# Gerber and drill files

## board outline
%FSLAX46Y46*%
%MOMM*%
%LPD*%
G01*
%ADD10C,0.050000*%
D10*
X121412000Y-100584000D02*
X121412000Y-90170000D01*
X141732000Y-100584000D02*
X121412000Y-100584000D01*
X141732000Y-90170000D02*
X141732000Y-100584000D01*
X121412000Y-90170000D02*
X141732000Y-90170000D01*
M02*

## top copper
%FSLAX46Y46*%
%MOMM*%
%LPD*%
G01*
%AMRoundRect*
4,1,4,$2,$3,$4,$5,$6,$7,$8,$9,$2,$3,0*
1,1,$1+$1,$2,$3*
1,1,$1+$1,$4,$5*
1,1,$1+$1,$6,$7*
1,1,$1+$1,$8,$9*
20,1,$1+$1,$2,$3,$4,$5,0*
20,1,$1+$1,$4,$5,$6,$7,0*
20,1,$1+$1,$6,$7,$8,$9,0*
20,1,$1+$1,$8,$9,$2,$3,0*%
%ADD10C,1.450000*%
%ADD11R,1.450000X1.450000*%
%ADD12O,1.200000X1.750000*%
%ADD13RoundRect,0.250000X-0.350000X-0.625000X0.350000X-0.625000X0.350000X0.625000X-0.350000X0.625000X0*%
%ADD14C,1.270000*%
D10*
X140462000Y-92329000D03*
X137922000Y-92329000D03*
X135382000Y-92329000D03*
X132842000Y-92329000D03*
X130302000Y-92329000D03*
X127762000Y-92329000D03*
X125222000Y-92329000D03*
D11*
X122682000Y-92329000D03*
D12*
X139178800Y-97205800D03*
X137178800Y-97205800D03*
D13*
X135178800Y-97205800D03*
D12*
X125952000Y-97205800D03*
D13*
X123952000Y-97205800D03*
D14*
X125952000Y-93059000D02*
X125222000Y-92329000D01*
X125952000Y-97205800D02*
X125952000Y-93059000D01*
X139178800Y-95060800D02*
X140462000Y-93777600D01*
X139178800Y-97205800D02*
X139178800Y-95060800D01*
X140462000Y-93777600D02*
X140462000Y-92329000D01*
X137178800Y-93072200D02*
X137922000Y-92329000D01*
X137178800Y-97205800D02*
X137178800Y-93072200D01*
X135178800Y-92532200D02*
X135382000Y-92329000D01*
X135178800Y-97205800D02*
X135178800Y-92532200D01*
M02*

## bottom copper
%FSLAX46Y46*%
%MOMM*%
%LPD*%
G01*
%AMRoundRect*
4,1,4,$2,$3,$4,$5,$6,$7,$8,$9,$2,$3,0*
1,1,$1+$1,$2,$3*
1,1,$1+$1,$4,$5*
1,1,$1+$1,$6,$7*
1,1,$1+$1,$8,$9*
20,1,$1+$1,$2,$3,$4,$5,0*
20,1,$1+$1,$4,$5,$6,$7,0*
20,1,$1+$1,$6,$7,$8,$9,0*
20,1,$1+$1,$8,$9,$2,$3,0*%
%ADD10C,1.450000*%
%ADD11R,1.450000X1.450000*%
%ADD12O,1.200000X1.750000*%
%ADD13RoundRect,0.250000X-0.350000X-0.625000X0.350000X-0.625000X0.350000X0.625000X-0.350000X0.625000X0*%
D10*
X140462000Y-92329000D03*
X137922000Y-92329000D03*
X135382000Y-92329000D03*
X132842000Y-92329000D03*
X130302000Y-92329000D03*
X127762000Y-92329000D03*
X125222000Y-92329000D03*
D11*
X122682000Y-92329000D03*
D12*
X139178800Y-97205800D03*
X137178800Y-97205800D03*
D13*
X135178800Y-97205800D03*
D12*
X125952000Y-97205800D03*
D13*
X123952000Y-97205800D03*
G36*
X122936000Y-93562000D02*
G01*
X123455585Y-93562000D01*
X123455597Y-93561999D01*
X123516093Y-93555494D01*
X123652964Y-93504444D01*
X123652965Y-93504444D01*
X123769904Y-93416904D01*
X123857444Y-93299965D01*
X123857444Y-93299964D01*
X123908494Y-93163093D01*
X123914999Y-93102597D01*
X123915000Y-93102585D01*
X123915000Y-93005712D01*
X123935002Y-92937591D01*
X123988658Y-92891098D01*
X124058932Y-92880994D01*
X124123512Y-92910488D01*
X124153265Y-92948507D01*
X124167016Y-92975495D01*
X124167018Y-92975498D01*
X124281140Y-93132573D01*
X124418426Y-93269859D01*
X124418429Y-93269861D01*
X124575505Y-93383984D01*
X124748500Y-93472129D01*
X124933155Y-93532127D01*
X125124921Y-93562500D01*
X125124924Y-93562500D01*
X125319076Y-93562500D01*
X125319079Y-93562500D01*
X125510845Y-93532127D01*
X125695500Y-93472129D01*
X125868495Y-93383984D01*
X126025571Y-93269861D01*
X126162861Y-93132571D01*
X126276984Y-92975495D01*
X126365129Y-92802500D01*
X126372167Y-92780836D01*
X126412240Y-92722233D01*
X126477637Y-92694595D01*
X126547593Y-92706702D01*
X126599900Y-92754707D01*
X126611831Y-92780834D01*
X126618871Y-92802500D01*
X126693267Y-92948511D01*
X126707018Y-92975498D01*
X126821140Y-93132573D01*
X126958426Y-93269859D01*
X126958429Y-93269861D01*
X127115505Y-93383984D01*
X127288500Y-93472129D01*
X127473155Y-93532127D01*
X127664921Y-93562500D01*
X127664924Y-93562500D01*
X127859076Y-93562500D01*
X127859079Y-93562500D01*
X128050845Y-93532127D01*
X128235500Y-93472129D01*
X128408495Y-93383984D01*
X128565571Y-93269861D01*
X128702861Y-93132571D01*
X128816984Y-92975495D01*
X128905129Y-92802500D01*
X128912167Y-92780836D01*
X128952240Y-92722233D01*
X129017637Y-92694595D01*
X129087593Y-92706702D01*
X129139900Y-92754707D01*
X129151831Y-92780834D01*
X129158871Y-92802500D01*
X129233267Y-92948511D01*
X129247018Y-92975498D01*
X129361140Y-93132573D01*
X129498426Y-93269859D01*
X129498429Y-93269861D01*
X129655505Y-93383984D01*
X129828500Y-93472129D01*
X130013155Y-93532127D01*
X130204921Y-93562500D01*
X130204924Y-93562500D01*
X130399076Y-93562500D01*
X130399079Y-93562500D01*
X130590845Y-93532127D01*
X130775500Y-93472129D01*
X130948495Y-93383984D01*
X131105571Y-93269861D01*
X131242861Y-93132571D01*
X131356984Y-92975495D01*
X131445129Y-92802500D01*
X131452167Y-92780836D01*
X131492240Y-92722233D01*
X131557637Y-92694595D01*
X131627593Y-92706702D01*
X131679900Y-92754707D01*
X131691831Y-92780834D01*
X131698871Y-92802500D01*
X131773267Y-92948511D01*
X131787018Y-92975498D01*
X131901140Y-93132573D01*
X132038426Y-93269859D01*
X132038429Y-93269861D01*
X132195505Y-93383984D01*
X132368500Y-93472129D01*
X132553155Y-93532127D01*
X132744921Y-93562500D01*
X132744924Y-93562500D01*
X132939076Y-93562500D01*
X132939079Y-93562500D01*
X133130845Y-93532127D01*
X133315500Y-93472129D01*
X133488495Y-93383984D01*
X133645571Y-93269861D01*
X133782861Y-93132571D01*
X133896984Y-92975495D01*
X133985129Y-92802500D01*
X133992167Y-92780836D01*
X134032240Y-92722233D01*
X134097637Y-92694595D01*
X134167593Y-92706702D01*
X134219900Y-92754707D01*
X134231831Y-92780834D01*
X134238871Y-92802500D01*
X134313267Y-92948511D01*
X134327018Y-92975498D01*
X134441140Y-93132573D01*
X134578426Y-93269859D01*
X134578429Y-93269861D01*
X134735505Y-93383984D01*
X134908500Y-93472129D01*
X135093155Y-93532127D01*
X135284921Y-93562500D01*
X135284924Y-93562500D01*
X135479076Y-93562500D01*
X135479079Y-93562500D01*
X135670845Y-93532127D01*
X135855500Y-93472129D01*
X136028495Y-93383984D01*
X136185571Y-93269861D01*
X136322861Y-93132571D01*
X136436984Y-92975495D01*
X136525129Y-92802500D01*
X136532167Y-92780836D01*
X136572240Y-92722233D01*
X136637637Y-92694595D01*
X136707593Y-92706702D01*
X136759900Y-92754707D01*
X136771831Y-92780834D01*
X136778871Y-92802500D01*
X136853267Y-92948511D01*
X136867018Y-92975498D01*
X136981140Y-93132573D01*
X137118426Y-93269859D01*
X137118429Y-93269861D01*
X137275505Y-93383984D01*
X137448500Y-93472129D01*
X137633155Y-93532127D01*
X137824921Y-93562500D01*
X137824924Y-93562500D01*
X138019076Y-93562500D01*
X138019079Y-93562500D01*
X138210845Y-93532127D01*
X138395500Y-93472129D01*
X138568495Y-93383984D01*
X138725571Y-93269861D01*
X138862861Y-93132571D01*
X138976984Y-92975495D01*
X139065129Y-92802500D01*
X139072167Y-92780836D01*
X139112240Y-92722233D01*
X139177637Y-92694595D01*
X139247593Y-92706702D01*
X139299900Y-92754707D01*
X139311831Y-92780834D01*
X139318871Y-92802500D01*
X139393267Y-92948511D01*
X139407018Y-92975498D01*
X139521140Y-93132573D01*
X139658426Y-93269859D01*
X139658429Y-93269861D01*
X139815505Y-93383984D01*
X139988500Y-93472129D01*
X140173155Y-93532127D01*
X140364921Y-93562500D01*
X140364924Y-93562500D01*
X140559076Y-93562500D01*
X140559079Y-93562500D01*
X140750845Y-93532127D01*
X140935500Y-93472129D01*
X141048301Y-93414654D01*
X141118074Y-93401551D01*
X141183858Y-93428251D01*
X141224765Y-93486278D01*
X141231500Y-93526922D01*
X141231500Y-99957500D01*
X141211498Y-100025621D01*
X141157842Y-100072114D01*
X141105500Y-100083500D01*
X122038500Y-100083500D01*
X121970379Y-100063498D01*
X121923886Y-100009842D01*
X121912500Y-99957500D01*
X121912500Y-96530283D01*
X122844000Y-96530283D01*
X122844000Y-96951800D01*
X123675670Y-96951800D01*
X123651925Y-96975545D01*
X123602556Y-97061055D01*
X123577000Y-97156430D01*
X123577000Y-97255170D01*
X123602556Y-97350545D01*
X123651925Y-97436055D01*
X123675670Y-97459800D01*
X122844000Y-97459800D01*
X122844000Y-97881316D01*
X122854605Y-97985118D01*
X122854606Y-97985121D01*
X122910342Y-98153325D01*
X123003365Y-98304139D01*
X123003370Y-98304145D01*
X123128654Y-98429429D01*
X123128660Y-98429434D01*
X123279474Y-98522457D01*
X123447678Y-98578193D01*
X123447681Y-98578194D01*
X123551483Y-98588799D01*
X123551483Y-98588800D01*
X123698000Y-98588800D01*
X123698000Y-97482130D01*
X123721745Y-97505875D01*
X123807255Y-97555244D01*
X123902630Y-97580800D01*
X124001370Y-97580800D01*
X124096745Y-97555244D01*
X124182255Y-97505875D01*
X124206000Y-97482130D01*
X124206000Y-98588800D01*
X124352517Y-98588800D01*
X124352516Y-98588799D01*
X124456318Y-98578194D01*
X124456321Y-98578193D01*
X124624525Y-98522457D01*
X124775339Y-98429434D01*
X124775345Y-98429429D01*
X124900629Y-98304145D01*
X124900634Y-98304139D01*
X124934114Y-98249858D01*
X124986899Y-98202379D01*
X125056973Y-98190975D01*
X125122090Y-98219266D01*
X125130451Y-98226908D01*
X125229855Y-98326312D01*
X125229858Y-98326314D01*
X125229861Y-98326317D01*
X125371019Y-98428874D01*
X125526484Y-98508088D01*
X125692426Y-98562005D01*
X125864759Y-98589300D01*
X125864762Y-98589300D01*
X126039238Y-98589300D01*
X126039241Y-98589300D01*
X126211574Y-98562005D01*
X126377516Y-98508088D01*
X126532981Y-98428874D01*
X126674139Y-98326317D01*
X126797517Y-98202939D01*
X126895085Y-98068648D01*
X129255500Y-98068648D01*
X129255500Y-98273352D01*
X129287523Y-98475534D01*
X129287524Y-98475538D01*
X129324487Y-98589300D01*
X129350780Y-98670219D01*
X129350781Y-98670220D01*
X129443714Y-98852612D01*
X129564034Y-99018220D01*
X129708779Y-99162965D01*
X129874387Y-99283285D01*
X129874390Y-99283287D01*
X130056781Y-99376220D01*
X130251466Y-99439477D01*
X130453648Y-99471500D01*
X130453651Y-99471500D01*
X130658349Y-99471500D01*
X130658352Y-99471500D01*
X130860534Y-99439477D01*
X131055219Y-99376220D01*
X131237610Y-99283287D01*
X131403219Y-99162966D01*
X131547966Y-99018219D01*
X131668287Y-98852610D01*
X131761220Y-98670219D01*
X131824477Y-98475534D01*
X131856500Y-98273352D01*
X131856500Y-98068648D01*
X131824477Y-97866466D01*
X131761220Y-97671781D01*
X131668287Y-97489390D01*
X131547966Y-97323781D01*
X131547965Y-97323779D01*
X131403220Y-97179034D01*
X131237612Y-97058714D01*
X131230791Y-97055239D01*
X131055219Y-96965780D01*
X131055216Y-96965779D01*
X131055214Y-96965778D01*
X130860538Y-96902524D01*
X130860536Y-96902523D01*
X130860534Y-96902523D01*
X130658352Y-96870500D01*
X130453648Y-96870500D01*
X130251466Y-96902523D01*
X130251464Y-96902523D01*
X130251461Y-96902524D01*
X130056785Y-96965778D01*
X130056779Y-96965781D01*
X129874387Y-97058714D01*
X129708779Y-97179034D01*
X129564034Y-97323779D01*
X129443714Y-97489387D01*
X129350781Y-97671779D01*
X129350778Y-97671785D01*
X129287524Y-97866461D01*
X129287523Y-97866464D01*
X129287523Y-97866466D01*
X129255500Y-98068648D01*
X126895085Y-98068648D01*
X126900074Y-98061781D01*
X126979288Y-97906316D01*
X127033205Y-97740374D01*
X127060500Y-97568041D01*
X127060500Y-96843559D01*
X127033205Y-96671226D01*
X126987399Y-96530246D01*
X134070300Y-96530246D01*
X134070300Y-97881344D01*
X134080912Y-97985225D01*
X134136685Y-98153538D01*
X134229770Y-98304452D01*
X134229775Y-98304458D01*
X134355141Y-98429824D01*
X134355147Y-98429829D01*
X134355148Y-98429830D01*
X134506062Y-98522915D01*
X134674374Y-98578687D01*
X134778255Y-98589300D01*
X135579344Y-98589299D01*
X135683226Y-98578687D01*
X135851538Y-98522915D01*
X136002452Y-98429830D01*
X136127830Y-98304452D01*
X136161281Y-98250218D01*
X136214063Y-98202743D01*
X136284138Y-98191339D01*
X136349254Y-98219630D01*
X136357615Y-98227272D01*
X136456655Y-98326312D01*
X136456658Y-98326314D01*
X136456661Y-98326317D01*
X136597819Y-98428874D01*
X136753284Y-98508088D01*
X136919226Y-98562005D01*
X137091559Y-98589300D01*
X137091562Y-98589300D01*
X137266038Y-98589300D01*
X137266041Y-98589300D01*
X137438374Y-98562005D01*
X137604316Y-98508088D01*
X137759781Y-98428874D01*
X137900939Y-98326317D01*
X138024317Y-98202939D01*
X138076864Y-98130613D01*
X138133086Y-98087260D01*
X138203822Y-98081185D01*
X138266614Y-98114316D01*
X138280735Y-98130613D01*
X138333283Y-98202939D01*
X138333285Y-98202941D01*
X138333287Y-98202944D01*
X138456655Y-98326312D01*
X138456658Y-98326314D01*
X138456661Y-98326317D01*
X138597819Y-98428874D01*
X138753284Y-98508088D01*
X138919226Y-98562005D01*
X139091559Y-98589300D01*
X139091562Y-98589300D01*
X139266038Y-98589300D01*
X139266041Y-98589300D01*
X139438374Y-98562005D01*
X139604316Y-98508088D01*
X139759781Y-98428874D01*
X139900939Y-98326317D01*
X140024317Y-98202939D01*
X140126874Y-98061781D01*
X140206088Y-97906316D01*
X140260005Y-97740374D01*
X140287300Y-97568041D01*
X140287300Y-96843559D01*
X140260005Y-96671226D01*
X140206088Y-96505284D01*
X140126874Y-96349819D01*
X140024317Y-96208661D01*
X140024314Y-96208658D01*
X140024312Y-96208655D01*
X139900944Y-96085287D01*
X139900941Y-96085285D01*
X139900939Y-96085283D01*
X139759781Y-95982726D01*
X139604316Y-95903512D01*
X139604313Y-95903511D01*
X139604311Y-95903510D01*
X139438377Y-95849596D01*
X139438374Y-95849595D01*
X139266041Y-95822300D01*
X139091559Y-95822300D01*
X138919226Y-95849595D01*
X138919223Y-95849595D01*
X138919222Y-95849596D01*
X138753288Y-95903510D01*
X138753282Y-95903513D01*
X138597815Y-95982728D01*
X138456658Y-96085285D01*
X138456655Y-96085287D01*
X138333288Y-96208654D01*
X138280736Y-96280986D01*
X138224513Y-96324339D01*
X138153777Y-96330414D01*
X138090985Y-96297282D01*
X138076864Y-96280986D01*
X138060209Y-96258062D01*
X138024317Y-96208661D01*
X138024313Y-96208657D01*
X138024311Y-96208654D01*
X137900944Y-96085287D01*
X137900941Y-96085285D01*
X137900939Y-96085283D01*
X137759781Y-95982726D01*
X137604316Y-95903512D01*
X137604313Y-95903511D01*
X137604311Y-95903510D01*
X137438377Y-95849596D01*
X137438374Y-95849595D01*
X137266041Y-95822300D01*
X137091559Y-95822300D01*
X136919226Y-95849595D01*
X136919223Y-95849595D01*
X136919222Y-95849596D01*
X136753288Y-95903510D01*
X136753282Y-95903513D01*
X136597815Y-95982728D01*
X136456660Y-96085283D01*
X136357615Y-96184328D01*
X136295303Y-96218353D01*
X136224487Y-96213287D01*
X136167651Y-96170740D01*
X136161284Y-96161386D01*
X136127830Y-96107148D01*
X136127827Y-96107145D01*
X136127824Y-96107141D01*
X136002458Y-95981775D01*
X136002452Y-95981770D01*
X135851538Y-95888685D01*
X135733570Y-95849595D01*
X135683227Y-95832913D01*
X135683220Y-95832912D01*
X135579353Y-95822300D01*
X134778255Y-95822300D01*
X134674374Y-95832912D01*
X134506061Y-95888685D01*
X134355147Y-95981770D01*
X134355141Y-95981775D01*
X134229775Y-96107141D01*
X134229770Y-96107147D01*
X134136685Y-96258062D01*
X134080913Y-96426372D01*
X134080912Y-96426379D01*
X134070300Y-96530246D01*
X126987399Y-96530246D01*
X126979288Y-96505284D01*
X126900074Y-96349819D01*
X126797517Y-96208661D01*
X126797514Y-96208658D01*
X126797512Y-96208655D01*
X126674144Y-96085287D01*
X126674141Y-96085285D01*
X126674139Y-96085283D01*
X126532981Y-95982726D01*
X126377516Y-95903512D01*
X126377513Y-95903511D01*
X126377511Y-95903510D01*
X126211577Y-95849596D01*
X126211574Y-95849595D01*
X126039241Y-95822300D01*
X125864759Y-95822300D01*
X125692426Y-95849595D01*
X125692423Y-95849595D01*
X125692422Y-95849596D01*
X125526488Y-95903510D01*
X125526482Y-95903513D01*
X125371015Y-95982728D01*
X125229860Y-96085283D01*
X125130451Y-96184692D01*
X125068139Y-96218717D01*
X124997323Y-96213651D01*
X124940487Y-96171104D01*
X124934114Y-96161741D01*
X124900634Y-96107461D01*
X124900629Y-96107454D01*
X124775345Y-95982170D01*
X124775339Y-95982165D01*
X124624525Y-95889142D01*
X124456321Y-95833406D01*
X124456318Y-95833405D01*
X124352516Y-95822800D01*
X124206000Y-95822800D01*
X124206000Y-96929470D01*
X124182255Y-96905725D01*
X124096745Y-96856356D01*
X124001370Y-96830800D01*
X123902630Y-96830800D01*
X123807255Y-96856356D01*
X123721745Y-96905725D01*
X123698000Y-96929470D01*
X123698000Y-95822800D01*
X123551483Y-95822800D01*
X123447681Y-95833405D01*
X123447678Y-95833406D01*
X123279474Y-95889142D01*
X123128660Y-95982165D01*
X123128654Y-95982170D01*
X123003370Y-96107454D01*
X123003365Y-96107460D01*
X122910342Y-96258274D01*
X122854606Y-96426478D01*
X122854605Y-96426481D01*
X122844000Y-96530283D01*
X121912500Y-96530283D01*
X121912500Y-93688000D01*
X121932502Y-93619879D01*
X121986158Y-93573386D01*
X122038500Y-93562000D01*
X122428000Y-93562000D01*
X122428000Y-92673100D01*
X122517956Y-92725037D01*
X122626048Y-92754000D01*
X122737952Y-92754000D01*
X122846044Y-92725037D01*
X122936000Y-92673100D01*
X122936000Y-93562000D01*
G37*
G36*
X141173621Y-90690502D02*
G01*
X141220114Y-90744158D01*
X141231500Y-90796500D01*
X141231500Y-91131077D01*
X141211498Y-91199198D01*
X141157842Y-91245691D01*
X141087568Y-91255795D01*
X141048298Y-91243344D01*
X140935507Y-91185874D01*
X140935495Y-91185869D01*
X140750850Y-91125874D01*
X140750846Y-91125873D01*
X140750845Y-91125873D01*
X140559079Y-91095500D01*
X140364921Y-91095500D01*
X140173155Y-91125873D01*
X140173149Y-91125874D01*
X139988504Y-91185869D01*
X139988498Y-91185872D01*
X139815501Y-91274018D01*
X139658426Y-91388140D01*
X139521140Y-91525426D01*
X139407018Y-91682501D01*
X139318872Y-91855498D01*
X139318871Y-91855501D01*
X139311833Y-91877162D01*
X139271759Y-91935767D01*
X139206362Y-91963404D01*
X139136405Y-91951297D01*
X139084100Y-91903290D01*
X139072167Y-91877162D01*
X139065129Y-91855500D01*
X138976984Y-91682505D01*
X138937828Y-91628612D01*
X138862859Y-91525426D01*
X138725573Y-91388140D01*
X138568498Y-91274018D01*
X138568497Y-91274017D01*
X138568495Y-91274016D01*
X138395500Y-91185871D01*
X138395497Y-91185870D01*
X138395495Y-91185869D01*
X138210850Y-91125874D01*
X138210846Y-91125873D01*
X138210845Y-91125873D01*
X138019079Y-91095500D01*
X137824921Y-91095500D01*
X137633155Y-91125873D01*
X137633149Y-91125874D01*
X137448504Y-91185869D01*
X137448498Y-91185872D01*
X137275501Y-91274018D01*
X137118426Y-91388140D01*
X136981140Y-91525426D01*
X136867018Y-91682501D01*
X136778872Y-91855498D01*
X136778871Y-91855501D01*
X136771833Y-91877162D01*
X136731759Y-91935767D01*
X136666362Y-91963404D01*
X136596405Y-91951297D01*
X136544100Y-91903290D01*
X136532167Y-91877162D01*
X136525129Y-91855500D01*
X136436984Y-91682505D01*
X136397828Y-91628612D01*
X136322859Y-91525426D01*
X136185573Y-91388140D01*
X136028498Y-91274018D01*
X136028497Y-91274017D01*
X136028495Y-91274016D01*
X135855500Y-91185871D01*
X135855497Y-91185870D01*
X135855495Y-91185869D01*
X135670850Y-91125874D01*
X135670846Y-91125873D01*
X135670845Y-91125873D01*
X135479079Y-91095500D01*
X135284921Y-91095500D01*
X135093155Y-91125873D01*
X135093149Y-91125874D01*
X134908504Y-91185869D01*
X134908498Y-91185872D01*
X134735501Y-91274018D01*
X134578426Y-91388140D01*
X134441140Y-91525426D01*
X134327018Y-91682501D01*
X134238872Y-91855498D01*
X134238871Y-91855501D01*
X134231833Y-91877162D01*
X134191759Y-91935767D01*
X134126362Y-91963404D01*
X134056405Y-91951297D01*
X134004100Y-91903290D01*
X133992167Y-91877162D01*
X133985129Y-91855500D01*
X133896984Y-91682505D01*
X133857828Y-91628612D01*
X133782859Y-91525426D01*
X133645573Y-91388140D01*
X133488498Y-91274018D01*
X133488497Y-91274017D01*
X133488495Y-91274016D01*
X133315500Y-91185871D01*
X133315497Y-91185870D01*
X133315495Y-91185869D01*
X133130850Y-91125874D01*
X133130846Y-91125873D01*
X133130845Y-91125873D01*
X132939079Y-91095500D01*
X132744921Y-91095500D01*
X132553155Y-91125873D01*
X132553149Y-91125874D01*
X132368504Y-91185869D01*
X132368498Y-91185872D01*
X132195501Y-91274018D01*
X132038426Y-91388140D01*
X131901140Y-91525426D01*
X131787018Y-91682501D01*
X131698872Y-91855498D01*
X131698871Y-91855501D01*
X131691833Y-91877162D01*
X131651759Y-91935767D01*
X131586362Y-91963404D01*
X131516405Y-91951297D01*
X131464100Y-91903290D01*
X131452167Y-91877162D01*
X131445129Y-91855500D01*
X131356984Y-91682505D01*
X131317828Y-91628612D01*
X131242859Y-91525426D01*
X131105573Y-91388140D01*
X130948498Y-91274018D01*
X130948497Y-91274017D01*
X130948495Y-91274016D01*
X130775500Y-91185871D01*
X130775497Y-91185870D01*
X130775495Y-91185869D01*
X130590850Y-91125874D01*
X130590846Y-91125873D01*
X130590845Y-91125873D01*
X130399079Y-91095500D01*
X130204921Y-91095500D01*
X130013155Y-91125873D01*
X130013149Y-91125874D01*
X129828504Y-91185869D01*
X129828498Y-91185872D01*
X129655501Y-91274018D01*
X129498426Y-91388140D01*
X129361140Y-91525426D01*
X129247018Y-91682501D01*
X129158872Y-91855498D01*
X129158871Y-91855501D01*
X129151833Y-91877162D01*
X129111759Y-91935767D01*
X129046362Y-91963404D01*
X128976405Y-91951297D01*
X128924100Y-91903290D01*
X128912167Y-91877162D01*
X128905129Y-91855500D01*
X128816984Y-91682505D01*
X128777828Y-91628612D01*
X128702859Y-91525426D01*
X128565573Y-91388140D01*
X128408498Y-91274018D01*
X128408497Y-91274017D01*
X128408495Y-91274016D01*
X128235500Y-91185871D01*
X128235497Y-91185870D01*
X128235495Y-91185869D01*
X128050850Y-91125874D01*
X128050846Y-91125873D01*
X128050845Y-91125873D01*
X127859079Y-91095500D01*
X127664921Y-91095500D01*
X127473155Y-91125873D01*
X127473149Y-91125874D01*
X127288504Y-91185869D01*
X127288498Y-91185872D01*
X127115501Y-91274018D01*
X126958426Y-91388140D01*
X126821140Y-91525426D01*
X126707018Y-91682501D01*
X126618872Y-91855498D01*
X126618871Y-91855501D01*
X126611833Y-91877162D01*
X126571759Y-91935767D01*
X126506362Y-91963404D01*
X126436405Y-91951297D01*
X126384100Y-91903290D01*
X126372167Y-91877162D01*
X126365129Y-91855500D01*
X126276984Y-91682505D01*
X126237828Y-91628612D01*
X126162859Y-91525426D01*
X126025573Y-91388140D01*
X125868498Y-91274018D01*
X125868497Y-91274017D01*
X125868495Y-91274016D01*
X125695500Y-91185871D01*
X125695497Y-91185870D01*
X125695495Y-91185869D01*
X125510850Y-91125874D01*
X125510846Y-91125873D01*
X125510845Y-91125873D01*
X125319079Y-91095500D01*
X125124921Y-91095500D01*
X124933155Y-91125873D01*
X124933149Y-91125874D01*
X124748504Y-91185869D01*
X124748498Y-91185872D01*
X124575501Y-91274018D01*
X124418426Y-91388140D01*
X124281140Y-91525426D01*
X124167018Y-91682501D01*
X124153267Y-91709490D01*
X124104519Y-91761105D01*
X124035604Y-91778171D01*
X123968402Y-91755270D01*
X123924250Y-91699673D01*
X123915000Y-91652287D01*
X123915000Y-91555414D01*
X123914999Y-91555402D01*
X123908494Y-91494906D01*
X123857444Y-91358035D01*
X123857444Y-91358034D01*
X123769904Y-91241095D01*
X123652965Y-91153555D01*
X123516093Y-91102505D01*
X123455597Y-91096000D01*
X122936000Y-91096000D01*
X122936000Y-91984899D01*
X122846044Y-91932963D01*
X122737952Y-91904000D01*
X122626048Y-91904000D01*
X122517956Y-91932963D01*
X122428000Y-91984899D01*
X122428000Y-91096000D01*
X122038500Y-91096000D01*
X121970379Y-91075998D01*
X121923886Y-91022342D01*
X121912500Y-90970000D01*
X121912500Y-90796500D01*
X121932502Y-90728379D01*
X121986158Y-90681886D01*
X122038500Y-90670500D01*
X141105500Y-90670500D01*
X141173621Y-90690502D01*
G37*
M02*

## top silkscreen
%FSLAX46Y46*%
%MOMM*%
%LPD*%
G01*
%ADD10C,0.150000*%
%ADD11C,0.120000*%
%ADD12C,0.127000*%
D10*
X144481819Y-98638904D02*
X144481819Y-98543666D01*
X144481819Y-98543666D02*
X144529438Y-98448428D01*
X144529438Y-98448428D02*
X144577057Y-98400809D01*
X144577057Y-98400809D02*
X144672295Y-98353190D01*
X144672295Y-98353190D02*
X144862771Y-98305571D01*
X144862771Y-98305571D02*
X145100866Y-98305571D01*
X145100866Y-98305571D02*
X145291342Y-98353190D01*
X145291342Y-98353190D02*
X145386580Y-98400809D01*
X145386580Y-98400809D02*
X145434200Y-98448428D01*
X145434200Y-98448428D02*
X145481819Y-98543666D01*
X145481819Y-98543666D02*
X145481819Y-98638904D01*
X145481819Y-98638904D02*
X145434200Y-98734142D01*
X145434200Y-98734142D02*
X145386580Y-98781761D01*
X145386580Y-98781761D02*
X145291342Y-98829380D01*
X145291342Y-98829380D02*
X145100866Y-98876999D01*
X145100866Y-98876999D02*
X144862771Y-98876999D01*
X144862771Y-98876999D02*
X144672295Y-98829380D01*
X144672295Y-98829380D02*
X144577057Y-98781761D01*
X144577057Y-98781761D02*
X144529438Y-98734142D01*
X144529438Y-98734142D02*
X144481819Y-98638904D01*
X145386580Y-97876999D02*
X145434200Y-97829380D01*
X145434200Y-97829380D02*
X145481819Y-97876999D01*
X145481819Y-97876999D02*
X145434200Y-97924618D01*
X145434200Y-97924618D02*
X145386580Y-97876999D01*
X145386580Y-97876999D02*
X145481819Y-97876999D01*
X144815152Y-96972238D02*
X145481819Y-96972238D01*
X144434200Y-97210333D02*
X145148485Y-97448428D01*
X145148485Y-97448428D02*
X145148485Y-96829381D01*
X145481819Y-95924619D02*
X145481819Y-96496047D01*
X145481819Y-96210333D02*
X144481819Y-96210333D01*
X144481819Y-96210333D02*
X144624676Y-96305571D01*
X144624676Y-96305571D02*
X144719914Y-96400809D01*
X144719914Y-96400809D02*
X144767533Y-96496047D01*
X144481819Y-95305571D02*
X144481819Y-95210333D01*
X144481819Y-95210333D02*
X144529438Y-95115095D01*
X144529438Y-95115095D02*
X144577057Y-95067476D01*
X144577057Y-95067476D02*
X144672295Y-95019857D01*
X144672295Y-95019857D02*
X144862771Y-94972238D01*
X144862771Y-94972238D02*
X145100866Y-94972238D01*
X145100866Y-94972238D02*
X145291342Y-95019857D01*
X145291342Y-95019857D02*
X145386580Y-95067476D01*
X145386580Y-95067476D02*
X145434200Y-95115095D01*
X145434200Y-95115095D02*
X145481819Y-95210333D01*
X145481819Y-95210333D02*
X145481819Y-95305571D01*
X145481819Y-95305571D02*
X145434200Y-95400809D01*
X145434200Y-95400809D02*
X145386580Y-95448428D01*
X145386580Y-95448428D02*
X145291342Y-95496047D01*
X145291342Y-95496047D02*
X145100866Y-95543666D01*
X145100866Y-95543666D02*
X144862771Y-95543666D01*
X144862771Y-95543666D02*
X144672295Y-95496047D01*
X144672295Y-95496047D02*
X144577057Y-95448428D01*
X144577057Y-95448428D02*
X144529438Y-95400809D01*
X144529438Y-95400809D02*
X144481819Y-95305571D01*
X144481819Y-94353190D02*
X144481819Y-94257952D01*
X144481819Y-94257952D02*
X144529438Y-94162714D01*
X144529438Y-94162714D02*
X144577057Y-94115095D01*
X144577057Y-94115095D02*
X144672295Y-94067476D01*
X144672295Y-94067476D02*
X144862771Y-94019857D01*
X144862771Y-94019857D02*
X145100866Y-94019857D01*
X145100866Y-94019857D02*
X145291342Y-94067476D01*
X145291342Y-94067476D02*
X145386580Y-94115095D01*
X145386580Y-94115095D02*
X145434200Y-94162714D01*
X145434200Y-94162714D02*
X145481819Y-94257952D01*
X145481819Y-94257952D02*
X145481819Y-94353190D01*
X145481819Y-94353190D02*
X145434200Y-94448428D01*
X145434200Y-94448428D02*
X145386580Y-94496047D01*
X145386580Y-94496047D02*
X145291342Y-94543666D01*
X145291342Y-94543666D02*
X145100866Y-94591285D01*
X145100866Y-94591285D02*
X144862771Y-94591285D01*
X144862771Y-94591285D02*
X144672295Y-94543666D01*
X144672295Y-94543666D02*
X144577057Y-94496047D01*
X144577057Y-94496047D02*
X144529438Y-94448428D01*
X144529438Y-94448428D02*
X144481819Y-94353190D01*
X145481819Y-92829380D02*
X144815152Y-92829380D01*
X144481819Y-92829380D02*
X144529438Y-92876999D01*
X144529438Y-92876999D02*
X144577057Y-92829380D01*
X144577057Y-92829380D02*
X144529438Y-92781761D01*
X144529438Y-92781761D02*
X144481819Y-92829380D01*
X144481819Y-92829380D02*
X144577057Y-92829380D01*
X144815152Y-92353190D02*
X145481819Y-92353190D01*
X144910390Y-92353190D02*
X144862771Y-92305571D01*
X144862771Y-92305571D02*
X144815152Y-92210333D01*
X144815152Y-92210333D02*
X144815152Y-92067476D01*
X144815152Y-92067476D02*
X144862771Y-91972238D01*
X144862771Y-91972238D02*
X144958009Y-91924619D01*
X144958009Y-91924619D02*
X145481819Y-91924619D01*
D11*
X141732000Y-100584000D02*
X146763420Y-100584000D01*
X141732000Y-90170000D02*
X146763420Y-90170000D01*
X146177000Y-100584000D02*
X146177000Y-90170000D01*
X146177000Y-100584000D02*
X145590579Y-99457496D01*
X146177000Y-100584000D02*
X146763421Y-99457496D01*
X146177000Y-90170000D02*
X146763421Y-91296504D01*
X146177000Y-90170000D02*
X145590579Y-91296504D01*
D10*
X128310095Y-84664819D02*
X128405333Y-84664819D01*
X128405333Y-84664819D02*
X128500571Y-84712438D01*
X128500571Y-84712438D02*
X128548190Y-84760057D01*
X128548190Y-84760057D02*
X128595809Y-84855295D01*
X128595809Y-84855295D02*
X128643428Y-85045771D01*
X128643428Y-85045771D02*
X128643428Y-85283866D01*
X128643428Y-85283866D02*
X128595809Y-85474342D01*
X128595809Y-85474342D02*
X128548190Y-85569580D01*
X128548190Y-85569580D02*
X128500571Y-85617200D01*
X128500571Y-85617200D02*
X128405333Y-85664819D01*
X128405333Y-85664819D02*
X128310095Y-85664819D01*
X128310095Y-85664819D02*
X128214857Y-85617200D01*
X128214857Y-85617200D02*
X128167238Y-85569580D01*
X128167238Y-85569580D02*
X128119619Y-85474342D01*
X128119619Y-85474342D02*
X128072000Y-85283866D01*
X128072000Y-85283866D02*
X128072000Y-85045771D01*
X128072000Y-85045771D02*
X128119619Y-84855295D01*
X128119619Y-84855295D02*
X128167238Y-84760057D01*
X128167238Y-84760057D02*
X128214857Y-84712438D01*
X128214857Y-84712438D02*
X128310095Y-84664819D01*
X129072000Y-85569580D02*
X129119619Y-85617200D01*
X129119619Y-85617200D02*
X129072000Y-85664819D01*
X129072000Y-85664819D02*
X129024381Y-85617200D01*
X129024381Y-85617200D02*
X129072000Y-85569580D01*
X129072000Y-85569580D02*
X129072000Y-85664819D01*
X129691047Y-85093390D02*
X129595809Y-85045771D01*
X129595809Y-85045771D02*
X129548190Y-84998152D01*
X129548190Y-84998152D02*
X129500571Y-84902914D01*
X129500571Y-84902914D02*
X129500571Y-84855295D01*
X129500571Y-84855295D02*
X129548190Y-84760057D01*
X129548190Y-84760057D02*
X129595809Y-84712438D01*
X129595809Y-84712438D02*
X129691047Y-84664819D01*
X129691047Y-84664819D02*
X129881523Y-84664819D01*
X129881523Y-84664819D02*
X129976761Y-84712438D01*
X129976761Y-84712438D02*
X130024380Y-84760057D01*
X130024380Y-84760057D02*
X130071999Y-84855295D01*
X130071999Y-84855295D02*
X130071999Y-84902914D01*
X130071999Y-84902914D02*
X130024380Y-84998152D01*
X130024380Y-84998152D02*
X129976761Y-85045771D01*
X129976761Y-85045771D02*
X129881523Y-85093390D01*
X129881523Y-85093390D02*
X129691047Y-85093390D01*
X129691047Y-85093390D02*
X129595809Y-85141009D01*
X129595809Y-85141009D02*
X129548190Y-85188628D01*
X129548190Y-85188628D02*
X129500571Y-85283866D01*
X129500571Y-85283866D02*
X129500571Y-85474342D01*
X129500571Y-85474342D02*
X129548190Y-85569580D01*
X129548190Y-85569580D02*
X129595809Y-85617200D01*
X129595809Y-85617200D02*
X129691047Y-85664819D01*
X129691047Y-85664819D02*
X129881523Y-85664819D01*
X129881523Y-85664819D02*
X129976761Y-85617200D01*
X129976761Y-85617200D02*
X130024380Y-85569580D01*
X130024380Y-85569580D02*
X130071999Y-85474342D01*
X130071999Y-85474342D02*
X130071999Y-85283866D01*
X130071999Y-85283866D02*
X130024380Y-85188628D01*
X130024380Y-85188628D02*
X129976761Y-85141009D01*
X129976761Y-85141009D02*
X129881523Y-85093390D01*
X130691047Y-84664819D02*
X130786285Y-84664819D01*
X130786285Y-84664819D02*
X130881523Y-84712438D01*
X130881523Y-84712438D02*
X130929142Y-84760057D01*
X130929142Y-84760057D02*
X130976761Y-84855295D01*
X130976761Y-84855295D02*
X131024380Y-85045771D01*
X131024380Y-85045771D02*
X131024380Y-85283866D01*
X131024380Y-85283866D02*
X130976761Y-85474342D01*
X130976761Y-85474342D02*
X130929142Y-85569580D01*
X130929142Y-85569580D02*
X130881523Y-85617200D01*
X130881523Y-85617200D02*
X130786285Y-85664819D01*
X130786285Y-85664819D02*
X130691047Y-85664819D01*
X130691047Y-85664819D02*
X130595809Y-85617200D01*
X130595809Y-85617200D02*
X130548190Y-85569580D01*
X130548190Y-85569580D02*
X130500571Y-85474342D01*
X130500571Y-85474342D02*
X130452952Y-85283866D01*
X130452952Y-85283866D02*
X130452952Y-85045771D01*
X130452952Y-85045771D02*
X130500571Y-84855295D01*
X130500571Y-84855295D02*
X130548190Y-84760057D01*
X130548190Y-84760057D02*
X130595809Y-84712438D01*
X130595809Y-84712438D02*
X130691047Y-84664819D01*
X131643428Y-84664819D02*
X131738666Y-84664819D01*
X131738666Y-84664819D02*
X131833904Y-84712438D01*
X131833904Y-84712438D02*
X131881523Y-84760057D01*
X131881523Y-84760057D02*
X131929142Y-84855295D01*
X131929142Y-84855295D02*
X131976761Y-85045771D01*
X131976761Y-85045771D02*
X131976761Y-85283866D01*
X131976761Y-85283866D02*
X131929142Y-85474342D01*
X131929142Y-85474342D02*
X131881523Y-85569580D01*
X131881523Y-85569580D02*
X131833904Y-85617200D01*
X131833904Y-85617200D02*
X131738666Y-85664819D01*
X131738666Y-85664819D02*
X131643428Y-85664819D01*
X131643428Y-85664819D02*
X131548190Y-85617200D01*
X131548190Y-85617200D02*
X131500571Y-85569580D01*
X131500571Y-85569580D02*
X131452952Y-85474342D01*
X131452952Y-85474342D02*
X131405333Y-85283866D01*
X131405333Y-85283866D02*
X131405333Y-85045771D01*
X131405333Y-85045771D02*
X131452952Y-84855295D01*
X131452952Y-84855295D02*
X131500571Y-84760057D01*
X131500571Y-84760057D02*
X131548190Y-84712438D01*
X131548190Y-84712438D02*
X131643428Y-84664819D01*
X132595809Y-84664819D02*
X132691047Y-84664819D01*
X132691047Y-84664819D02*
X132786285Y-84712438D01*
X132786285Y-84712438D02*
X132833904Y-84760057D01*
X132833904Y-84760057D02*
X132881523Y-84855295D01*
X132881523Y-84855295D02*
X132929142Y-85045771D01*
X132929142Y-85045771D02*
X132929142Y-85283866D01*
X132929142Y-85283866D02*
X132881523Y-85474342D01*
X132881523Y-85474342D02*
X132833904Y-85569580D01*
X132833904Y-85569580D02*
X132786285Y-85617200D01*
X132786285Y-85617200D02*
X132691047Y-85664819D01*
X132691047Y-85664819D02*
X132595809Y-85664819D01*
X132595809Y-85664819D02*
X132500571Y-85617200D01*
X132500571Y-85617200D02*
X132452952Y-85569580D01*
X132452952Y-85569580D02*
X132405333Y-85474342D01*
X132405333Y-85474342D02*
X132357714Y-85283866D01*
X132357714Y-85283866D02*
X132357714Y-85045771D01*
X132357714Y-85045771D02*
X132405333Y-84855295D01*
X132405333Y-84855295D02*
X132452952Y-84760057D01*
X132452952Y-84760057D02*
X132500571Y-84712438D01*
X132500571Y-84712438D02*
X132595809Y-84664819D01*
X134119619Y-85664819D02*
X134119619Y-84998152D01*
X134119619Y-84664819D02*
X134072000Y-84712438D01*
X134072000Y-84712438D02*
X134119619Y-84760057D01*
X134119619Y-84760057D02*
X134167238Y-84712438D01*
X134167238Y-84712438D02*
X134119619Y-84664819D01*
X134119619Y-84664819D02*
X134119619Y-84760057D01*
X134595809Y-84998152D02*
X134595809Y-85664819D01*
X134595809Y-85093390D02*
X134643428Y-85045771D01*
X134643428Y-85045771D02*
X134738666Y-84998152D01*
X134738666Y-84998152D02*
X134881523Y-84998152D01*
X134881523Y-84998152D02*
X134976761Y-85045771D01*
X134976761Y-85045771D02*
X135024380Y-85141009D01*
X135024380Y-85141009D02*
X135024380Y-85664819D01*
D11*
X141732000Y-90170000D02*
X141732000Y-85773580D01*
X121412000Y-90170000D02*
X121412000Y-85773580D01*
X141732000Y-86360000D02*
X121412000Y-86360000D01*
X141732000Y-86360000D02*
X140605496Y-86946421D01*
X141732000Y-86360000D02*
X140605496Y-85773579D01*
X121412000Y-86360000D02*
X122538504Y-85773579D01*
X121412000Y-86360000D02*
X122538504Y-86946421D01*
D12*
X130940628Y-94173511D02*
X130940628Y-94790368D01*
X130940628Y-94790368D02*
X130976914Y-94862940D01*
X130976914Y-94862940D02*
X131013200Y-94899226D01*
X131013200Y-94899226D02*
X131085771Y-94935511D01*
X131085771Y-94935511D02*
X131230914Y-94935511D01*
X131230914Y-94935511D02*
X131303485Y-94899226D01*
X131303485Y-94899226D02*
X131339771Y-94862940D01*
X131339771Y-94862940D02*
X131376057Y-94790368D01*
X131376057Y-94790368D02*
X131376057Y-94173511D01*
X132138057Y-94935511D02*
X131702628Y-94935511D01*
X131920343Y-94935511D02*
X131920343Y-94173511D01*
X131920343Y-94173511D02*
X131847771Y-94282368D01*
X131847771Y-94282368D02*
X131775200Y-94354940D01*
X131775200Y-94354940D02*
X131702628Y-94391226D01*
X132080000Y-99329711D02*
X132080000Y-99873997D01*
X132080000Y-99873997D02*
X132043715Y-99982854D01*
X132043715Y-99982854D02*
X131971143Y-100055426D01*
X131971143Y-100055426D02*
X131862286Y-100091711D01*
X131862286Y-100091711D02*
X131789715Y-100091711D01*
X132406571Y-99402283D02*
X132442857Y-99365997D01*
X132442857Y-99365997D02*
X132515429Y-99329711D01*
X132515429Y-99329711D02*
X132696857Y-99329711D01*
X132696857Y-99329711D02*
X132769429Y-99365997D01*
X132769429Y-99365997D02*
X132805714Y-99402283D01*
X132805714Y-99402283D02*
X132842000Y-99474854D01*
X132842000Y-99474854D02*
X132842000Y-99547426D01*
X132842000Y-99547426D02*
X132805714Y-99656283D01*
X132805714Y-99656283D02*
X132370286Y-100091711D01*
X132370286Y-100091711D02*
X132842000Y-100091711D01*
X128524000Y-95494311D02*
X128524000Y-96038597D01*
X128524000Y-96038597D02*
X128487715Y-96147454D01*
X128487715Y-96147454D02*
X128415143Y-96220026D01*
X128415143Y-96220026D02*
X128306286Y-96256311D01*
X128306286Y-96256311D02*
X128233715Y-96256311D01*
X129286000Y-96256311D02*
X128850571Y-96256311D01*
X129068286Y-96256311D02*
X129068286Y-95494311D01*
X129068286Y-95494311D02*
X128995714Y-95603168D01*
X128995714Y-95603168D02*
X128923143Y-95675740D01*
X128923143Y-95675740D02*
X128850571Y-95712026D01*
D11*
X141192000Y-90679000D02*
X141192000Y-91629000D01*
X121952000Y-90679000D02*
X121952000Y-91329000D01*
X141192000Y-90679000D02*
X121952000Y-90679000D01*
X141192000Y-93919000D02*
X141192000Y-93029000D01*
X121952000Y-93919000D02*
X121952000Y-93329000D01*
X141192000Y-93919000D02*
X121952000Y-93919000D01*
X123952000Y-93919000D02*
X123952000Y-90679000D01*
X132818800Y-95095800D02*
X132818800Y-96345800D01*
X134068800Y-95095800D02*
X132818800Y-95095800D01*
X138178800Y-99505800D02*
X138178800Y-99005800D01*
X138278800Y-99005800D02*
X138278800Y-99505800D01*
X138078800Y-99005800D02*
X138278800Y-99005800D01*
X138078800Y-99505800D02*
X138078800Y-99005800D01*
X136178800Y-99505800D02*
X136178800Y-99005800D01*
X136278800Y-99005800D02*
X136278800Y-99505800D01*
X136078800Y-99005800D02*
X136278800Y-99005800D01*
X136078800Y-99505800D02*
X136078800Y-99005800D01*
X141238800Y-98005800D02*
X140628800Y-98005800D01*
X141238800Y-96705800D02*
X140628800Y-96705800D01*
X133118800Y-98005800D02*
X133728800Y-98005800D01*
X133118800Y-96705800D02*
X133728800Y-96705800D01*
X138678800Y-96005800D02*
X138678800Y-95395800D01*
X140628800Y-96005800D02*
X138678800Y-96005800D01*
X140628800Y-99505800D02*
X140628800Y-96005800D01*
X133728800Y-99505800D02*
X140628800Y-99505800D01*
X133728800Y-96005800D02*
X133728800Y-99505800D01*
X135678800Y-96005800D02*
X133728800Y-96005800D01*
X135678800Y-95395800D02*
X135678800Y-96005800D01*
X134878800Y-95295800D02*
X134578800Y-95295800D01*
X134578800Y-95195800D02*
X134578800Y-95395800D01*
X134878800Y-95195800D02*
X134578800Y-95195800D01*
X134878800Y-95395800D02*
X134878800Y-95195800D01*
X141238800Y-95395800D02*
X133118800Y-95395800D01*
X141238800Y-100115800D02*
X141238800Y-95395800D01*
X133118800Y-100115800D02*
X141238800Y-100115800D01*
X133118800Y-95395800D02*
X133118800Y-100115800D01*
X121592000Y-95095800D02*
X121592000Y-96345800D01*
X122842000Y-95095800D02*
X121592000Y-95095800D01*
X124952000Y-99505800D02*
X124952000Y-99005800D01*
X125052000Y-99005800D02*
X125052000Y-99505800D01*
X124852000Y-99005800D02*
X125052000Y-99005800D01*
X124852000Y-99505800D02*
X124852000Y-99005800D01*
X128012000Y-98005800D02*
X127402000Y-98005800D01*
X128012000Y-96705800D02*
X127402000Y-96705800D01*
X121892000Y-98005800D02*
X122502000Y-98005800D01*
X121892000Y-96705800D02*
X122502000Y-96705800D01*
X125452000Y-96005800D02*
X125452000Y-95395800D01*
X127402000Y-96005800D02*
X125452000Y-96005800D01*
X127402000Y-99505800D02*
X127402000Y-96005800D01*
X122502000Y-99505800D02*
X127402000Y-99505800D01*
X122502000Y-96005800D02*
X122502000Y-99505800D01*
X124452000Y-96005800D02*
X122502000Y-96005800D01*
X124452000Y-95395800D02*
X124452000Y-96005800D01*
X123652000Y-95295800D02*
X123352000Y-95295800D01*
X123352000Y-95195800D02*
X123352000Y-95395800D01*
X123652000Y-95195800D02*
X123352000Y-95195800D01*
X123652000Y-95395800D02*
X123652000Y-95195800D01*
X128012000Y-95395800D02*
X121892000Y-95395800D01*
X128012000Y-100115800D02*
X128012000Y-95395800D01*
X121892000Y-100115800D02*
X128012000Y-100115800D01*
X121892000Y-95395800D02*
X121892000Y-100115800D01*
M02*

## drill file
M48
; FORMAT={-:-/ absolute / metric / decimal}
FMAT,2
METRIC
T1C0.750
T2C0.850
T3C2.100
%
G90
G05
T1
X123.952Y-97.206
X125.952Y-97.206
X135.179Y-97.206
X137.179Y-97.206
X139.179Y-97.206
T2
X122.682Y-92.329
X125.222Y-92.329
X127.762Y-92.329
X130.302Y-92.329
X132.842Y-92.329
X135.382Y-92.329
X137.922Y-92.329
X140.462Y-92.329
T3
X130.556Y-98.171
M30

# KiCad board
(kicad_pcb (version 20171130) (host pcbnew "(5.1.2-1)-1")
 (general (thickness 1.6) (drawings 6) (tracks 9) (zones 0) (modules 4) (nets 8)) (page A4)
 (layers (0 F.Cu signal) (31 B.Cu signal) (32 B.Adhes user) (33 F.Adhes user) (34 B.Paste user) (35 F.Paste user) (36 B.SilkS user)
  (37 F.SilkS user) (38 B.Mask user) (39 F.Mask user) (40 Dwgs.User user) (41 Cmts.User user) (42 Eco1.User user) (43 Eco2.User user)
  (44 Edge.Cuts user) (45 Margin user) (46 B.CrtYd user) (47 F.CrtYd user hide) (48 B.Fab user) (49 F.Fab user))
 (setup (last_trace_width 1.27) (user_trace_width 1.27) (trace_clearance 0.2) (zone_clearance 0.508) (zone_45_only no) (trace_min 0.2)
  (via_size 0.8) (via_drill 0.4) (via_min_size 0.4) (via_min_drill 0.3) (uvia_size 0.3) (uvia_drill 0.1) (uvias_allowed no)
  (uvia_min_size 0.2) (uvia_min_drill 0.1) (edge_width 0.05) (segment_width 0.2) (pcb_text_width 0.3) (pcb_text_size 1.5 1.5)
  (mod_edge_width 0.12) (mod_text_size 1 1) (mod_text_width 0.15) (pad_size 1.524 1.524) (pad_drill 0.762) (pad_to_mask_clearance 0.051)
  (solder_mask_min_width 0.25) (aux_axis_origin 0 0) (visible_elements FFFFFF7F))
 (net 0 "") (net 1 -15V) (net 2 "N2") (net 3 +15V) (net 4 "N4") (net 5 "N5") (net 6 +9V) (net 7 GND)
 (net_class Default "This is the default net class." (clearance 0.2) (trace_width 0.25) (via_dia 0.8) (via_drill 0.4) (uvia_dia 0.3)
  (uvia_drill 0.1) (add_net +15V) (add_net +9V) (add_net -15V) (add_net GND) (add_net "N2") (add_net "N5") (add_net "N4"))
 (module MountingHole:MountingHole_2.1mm (layer F.Cu) (at 130.556 98.171)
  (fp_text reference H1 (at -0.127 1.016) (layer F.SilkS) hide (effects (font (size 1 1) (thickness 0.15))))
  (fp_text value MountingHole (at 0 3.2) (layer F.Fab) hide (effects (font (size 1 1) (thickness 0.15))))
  (pad "" np_thru_hole circle (at 0 0) (size 2.1 2.1) (drill 2.1) (layers *.Cu *.Mask)))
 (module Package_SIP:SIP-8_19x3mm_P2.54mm (layer F.Cu) (at 122.682 92.329)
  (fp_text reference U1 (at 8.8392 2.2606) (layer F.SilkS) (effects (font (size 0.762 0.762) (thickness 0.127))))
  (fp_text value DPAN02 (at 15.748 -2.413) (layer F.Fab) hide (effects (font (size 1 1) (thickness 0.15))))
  (fp_line (start 18.51 -1.65) (end 18.51 -0.7) (layer F.SilkS) (width 0.12))
  (fp_line (start -0.73 -1.65) (end -0.73 -1) (layer F.SilkS) (width 0.12))
  (fp_line (start 18.51 -1.65) (end -0.73 -1.65) (layer F.SilkS) (width 0.12))
  (fp_line (start 18.51 1.59) (end 18.51 0.7) (layer F.SilkS) (width 0.12))
  (fp_line (start -0.73 1.59) (end -0.73 1) (layer F.SilkS) (width 0.12))
  (fp_line (start 18.51 1.59) (end -0.73 1.59) (layer F.SilkS) (width 0.12))
  (fp_line (start 1.27 1.59) (end 1.27 -1.65) (layer F.SilkS) (width 0.12))
  (pad 8 thru_hole circle (at 17.78 0 90) (size 1.45 1.45) (drill 0.85) (layers *.Cu *.Mask) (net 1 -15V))
  (pad 7 thru_hole circle (at 15.24 0 90) (size 1.45 1.45) (drill 0.85) (layers *.Cu *.Mask) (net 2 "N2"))
  (pad 6 thru_hole circle (at 12.7 0 90) (size 1.45 1.45) (drill 0.85) (layers *.Cu *.Mask) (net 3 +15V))
  (pad 5 thru_hole circle (at 10.16 0 90) (size 1.45 1.45) (drill 0.85) (layers *.Cu *.Mask) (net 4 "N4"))
  (pad 4 thru_hole circle (at 7.62 0 90) (size 1.45 1.45) (drill 0.85) (layers *.Cu *.Mask))
  (pad 3 thru_hole circle (at 5.08 0 90) (size 1.45 1.45) (drill 0.85) (layers *.Cu *.Mask) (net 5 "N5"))
  (pad 2 thru_hole circle (at 2.54 0 90) (size 1.45 1.45) (drill 0.85) (layers *.Cu *.Mask) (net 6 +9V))
  (pad 1 thru_hole rect (at 0 0 90) (size 1.45 1.45) (drill 0.85) (layers *.Cu *.Mask) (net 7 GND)))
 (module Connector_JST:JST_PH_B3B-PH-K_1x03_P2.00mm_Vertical (layer F.Cu) (at 135.1788 97.2058)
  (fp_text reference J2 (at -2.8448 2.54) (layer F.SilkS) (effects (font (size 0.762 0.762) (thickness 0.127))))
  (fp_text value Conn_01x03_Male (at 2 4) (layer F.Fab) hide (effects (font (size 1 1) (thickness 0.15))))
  (fp_line (start -2.36 -2.11) (end -2.36 -0.86) (layer F.SilkS) (width 0.12))
  (fp_line (start -1.11 -2.11) (end -2.36 -2.11) (layer F.SilkS) (width 0.12))
  (fp_line (start 3 2.3) (end 3 1.8) (layer F.SilkS) (width 0.12))
  (fp_line (start 3.1 1.8) (end 3.1 2.3) (layer F.SilkS) (width 0.12))
  (fp_line (start 2.9 1.8) (end 3.1 1.8) (layer F.SilkS) (width 0.12))
  (fp_line (start 2.9 2.3) (end 2.9 1.8) (layer F.SilkS) (width 0.12))
  (fp_line (start 1 2.3) (end 1 1.8) (layer F.SilkS) (width 0.12))
  (fp_line (start 1.1 1.8) (end 1.1 2.3) (layer F.SilkS) (width 0.12))
  (fp_line (start 0.9 1.8) (end 1.1 1.8) (layer F.SilkS) (width 0.12))
  (fp_line (start 0.9 2.3) (end 0.9 1.8) (layer F.SilkS) (width 0.12))
  (fp_line (start 6.06 0.8) (end 5.45 0.8) (layer F.SilkS) (width 0.12))
  (fp_line (start 6.06 -0.5) (end 5.45 -0.5) (layer F.SilkS) (width 0.12))
  (fp_line (start -2.06 0.8) (end -1.45 0.8) (layer F.SilkS) (width 0.12))
  (fp_line (start -2.06 -0.5) (end -1.45 -0.5) (layer F.SilkS) (width 0.12))
  (fp_line (start 3.5 -1.2) (end 3.5 -1.81) (layer F.SilkS) (width 0.12))
  (fp_line (start 5.45 -1.2) (end 3.5 -1.2) (layer F.SilkS) (width 0.12))
  (fp_line (start 5.45 2.3) (end 5.45 -1.2) (layer F.SilkS) (width 0.12))
  (fp_line (start -1.45 2.3) (end 5.45 2.3) (layer F.SilkS) (width 0.12))
  (fp_line (start -1.45 -1.2) (end -1.45 2.3) (layer F.SilkS) (width 0.12))
  (fp_line (start 0.5 -1.2) (end -1.45 -1.2) (layer F.SilkS) (width 0.12))
  (fp_line (start 0.5 -1.81) (end 0.5 -1.2) (layer F.SilkS) (width 0.12))
  (fp_line (start -0.3 -1.91) (end -0.6 -1.91) (layer F.SilkS) (width 0.12))
  (fp_line (start -0.6 -2.01) (end -0.6 -1.81) (layer F.SilkS) (width 0.12))
  (fp_line (start -0.3 -2.01) (end -0.6 -2.01) (layer F.SilkS) (width 0.12))
  (fp_line (start -0.3 -1.81) (end -0.3 -2.01) (layer F.SilkS) (width 0.12))
  (fp_line (start 6.06 -1.81) (end -2.06 -1.81) (layer F.SilkS) (width 0.12))
  (fp_line (start 6.06 2.91) (end 6.06 -1.81) (layer F.SilkS) (width 0.12))
  (fp_line (start -2.06 2.91) (end 6.06 2.91) (layer F.SilkS) (width 0.12))
  (fp_line (start -2.06 -1.81) (end -2.06 2.91) (layer F.SilkS) (width 0.12))
  (pad 3 thru_hole oval (at 4 0) (size 1.2 1.75) (drill 0.75) (layers *.Cu *.Mask) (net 1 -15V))
  (pad 2 thru_hole oval (at 2 0) (size 1.2 1.75) (drill 0.75) (layers *.Cu *.Mask) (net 2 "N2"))
  (pad 1 thru_hole roundrect (at 0 0) (size 1.2 1.75) (drill 0.75) (layers *.Cu *.Mask) (roundrect_rratio 0.208333) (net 3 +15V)))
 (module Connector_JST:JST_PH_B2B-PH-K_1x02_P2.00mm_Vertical (layer F.Cu) (at 123.952 97.2058)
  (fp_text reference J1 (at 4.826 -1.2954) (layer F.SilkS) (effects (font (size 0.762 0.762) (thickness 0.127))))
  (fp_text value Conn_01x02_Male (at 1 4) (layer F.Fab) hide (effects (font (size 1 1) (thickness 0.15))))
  (fp_line (start -2.36 -2.11) (end -2.36 -0.86) (layer F.SilkS) (width 0.12))
  (fp_line (start -1.11 -2.11) (end -2.36 -2.11) (layer F.SilkS) (width 0.12))
  (fp_line (start 1 2.3) (end 1 1.8) (layer F.SilkS) (width 0.12))
  (fp_line (start 1.1 1.8) (end 1.1 2.3) (layer F.SilkS) (width 0.12))
  (fp_line (start 0.9 1.8) (end 1.1 1.8) (layer F.SilkS) (width 0.12))
  (fp_line (start 0.9 2.3) (end 0.9 1.8) (layer F.SilkS) (width 0.12))
  (fp_line (start 4.06 0.8) (end 3.45 0.8) (layer F.SilkS) (width 0.12))
  (fp_line (start 4.06 -0.5) (end 3.45 -0.5) (layer F.SilkS) (width 0.12))
  (fp_line (start -2.06 0.8) (end -1.45 0.8) (layer F.SilkS) (width 0.12))
  (fp_line (start -2.06 -0.5) (end -1.45 -0.5) (layer F.SilkS) (width 0.12))
  (fp_line (start 1.5 -1.2) (end 1.5 -1.81) (layer F.SilkS) (width 0.12))
  (fp_line (start 3.45 -1.2) (end 1.5 -1.2) (layer F.SilkS) (width 0.12))
  (fp_line (start 3.45 2.3) (end 3.45 -1.2) (layer F.SilkS) (width 0.12))
  (fp_line (start -1.45 2.3) (end 3.45 2.3) (layer F.SilkS) (width 0.12))
  (fp_line (start -1.45 -1.2) (end -1.45 2.3) (layer F.SilkS) (width 0.12))
  (fp_line (start 0.5 -1.2) (end -1.45 -1.2) (layer F.SilkS) (width 0.12))
  (fp_line (start 0.5 -1.81) (end 0.5 -1.2) (layer F.SilkS) (width 0.12))
  (fp_line (start -0.3 -1.91) (end -0.6 -1.91) (layer F.SilkS) (width 0.12))
  (fp_line (start -0.6 -2.01) (end -0.6 -1.81) (layer F.SilkS) (width 0.12))
  (fp_line (start -0.3 -2.01) (end -0.6 -2.01) (layer F.SilkS) (width 0.12))
  (fp_line (start -0.3 -1.81) (end -0.3 -2.01) (layer F.SilkS) (width 0.12))
  (fp_line (start 4.06 -1.81) (end -2.06 -1.81) (layer F.SilkS) (width 0.12))
  (fp_line (start 4.06 2.91) (end 4.06 -1.81) (layer F.SilkS) (width 0.12))
  (fp_line (start -2.06 2.91) (end 4.06 2.91) (layer F.SilkS) (width 0.12))
  (fp_line (start -2.06 -1.81) (end -2.06 2.91) (layer F.SilkS) (width 0.12))
  (pad 2 thru_hole oval (at 2 0) (size 1.2 1.75) (drill 0.75) (layers *.Cu *.Mask) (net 6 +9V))
  (pad 1 thru_hole roundrect (at 0 0) (size 1.2 1.75) (drill 0.75) (layers *.Cu *.Mask) (roundrect_rratio 0.208333) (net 7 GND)))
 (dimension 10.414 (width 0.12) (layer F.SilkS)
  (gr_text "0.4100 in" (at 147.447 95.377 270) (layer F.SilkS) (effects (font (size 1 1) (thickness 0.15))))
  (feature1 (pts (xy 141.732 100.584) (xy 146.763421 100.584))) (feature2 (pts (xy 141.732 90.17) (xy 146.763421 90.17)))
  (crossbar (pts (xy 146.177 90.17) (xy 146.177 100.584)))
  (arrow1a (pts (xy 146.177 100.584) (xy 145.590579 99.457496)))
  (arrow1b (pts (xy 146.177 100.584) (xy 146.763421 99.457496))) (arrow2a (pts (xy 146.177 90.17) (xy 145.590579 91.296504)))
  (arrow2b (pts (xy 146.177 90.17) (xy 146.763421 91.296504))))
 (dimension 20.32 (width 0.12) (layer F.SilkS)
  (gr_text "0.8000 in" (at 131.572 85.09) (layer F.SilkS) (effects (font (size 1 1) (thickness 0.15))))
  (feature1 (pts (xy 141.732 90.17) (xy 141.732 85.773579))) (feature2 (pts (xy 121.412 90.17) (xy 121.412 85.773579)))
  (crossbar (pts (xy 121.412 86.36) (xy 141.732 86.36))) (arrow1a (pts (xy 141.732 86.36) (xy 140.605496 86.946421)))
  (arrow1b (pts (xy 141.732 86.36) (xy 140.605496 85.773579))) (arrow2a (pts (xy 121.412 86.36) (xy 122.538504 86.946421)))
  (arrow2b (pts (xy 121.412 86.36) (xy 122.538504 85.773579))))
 (gr_line (start 121.412 100.584) (end 121.412 90.17) (layer Edge.Cuts) (width 0.05))
 (gr_line (start 141.732 100.584) (end 121.412 100.584) (layer Edge.Cuts) (width 0.05))
 (gr_line (start 141.732 90.17) (end 141.732 100.584) (layer Edge.Cuts) (width 0.05))
 (gr_line (start 121.412 90.17) (end 141.732 90.17) (layer Edge.Cuts) (width 0.05))
 (segment (start 125.952 93.059) (end 125.222 92.329) (width 1.27) (layer F.Cu) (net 6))
 (segment (start 125.952 97.2058) (end 125.952 93.059) (width 1.27) (layer F.Cu) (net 6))
 (segment (start 139.1788 95.0608) (end 140.462 93.7776) (width 1.27) (layer F.Cu) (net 1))
 (segment (start 139.1788 97.2058) (end 139.1788 95.0608) (width 1.27) (layer F.Cu) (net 1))
 (segment (start 140.462 93.7776) (end 140.462 92.329) (width 1.27) (layer F.Cu) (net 1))
 (segment (start 137.1788 93.0722) (end 137.922 92.329) (width 1.27) (layer F.Cu) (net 2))
 (segment (start 137.1788 97.2058) (end 137.1788 93.0722) (width 1.27) (layer F.Cu) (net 2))
 (segment (start 135.1788 92.5322) (end 135.382 92.329) (width 1.27) (layer F.Cu) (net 3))
 (segment (start 135.1788 97.2058) (end 135.1788 92.5322) (width 1.27) (layer F.Cu) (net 3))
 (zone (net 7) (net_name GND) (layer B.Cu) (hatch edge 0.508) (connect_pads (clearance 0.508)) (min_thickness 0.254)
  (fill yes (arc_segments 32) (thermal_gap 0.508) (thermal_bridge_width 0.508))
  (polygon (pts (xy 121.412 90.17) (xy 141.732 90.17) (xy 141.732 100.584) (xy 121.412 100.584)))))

